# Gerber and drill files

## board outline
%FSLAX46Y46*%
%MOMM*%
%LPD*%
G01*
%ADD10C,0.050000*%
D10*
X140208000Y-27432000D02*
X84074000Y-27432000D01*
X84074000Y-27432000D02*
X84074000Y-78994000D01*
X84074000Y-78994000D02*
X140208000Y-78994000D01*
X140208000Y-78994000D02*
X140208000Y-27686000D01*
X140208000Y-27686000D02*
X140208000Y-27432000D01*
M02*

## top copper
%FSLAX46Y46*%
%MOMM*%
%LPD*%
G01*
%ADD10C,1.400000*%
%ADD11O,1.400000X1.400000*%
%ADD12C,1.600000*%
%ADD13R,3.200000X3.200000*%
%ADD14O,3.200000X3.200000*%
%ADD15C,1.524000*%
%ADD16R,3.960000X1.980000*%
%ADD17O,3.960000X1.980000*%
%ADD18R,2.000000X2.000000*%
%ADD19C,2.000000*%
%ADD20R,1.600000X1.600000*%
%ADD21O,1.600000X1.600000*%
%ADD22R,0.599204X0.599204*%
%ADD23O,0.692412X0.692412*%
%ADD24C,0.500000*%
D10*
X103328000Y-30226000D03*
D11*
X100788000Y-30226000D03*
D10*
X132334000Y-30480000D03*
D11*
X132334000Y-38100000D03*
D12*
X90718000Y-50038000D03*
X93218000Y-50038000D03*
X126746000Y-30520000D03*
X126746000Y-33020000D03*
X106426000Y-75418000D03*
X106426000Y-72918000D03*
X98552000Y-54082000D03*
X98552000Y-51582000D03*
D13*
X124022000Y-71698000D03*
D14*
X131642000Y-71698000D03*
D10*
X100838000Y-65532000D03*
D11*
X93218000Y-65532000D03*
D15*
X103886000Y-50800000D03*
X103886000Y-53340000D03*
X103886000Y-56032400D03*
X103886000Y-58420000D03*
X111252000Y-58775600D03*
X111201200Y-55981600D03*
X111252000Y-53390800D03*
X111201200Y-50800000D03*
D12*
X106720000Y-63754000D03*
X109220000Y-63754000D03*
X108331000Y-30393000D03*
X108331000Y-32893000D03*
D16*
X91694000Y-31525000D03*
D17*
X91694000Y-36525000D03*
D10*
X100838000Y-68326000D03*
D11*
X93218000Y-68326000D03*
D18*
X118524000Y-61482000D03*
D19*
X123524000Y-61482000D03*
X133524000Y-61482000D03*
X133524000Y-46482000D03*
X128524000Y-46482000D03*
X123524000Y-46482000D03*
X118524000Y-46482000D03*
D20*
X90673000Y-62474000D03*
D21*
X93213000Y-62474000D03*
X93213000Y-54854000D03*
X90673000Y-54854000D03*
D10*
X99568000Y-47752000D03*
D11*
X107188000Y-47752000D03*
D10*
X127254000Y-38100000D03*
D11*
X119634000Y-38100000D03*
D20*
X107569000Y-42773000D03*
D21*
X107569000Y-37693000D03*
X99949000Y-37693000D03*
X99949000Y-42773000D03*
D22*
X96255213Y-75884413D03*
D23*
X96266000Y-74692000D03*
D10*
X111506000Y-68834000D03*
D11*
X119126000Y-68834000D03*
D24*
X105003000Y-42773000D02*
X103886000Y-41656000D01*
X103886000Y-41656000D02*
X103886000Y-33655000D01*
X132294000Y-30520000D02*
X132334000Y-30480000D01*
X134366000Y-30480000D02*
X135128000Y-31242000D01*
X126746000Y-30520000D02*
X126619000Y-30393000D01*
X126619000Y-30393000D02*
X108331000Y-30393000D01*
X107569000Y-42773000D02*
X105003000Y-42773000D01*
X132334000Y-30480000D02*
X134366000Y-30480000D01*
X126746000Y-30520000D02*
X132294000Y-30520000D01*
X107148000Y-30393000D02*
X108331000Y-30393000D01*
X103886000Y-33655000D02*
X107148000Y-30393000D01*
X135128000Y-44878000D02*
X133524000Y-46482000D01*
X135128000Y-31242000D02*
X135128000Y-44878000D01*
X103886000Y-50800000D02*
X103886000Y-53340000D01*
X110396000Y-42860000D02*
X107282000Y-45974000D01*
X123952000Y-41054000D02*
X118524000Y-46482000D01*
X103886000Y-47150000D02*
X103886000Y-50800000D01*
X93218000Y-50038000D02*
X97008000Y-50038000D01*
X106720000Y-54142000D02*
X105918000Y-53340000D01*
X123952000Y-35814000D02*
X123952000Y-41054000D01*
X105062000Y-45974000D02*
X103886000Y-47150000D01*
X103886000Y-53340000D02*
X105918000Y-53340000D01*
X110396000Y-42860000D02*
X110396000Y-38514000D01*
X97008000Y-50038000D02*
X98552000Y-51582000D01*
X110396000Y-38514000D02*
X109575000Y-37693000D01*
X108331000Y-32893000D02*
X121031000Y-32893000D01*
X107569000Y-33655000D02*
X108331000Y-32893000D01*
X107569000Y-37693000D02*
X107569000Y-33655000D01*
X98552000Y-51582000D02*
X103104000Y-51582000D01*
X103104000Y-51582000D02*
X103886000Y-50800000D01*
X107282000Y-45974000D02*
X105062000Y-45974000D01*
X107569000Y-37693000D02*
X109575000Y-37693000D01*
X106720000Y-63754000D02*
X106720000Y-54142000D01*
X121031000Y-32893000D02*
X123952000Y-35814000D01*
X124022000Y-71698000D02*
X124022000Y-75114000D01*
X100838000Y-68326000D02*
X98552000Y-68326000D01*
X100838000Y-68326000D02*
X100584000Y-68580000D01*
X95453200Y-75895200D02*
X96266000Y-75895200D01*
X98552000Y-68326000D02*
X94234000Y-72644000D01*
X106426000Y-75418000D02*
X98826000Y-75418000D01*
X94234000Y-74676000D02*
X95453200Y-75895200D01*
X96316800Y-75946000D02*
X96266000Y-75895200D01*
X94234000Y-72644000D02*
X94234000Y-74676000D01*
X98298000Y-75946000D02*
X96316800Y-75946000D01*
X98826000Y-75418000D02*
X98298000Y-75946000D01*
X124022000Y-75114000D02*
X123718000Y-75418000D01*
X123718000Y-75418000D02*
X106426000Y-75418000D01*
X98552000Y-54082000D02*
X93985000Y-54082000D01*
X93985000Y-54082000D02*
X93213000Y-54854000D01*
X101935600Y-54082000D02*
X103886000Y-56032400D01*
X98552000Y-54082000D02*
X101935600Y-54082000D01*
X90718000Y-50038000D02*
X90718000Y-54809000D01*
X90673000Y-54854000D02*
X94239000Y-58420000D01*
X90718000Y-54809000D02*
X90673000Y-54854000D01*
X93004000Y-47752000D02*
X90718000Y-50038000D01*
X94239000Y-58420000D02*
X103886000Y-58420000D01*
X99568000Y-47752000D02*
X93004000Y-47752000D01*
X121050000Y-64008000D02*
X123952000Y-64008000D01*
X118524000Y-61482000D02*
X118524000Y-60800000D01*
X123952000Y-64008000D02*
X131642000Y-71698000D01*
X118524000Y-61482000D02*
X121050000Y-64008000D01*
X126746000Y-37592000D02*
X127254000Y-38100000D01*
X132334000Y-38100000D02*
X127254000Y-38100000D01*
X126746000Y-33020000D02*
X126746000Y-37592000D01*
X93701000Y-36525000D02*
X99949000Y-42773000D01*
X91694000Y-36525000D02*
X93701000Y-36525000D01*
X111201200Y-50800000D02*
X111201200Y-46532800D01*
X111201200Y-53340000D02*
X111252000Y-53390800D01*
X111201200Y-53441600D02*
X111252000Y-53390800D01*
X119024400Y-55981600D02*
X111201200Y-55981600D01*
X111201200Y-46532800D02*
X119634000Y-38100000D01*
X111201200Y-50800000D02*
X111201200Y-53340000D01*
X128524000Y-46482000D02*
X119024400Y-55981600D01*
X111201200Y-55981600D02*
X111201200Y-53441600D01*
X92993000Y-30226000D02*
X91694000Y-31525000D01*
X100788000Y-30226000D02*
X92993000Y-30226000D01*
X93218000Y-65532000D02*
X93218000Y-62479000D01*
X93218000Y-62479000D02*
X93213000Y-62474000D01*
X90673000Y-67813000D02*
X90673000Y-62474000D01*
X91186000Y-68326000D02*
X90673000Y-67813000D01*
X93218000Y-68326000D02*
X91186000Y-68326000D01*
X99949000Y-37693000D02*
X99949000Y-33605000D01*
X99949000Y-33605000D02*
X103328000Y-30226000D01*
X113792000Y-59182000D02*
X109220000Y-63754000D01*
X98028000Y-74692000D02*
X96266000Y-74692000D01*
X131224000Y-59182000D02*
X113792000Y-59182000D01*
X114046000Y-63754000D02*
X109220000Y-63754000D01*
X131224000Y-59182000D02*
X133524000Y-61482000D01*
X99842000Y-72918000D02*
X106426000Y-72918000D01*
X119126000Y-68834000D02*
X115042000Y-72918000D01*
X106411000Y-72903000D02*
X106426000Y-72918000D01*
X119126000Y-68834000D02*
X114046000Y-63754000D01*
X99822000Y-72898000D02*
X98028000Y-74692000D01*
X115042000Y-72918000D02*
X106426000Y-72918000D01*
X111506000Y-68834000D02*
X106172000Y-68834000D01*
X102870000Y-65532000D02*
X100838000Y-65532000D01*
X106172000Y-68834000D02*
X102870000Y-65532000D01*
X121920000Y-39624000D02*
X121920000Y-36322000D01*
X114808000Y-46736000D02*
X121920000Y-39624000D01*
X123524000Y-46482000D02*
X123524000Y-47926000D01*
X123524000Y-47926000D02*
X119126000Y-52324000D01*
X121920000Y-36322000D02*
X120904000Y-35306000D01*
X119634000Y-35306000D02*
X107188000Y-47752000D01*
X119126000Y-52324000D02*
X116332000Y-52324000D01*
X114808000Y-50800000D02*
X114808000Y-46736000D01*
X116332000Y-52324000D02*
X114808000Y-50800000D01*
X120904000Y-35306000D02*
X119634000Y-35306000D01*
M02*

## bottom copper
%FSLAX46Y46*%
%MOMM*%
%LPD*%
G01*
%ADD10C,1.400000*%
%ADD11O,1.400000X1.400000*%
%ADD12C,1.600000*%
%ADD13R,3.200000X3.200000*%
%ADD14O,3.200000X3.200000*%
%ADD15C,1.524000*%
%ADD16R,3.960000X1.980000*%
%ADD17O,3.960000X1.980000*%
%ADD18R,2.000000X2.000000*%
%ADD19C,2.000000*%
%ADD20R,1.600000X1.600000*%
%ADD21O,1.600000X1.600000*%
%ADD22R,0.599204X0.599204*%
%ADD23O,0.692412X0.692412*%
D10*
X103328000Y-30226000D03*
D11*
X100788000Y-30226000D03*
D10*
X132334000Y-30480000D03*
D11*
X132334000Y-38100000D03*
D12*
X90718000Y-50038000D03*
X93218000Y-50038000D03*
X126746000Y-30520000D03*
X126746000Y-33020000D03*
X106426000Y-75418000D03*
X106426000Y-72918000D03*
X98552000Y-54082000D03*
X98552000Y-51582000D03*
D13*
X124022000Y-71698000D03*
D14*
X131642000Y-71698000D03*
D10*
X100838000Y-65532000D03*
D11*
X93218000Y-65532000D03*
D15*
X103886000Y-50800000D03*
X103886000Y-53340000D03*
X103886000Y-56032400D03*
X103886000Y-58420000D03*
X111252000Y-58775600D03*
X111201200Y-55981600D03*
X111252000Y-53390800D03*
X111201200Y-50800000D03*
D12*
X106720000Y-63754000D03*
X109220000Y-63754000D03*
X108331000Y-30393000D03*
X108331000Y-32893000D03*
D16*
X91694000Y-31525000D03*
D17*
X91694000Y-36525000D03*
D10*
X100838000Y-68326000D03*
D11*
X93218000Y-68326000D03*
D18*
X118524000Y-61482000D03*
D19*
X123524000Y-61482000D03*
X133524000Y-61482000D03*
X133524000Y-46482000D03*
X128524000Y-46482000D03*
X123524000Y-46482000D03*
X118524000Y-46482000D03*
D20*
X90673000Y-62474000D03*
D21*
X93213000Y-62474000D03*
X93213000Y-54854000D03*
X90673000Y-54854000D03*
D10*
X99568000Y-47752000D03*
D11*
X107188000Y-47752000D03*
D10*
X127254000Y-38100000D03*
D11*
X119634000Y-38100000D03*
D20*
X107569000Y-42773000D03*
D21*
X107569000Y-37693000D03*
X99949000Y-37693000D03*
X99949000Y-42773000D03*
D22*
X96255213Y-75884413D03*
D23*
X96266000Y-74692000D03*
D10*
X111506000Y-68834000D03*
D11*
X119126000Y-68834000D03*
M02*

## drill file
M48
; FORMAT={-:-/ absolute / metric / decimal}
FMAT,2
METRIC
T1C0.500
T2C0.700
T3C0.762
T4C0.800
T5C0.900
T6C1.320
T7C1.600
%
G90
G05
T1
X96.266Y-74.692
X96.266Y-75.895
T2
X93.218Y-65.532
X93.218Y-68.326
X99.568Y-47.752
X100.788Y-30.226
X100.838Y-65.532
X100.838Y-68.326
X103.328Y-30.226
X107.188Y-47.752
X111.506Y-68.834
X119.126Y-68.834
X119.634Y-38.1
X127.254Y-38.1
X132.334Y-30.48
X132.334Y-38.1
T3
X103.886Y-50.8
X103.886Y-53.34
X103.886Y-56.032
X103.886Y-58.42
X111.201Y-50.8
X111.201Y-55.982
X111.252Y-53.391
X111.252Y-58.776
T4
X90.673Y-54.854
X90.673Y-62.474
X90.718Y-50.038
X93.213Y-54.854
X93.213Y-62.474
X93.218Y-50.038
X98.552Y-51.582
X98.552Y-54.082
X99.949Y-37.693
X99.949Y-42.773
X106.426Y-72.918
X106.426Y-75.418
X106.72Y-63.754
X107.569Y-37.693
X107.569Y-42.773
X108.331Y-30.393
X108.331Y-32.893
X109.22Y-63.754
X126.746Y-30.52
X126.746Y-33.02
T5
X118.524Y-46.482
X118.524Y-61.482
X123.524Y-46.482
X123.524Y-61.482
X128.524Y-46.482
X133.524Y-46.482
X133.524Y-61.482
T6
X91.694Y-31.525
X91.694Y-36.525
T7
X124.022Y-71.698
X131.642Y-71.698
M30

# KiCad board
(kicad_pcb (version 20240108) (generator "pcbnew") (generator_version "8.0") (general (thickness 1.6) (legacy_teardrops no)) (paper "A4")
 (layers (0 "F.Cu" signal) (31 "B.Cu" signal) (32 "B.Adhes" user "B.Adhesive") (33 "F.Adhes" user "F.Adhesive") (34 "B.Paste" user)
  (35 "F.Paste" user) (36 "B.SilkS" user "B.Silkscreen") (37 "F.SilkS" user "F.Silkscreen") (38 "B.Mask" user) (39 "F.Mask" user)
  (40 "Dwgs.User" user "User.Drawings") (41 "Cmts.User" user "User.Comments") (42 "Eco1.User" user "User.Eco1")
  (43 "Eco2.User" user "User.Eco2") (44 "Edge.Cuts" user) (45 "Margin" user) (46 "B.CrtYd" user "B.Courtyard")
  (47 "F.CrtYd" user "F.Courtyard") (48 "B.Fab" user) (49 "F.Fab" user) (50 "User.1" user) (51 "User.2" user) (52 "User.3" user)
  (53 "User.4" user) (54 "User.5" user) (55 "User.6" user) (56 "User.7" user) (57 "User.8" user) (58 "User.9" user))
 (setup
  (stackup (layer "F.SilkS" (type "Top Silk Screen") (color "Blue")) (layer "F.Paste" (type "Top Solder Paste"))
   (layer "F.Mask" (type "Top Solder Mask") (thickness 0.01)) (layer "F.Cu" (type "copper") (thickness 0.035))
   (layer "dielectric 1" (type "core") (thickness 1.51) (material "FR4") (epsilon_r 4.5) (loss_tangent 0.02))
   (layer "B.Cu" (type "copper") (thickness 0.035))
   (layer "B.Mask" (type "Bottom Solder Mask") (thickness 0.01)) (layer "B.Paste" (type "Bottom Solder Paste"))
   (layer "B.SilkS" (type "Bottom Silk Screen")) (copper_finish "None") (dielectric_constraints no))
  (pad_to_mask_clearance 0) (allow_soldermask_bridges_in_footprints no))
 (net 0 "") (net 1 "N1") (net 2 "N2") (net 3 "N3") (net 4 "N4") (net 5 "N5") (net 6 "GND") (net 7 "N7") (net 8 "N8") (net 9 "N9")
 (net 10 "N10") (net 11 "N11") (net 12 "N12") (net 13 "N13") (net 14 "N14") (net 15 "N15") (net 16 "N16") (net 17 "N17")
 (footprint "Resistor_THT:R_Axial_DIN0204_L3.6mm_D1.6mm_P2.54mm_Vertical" (layer "F.Cu") (at 103.328 30.226 180)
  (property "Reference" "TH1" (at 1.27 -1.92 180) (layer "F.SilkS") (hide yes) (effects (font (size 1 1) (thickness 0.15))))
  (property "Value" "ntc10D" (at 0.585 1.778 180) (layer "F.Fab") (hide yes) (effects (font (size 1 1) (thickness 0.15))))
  (pad "1" thru_hole circle (at 0 0 180) (size 1.4 1.4) (drill 0.7) (layers "*.Cu" "*.Mask") (remove_unused_layers no) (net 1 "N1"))
  (pad "2" thru_hole oval (at 2.54 0 180) (size 1.4 1.4) (drill 0.7) (layers "*.Cu" "*.Mask") (remove_unused_layers no) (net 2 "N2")))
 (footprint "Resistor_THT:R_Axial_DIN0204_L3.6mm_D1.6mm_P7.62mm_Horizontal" (layer "F.Cu") (at 132.334 30.48 -90)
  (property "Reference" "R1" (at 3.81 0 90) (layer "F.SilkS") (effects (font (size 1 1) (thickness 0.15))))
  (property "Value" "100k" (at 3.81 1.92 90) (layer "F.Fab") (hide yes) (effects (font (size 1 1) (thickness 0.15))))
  (pad "1" thru_hole circle (at 0 0 270) (size 1.4 1.4) (drill 0.7) (layers "*.Cu" "*.Mask") (remove_unused_layers no) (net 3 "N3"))
  (pad "2" thru_hole oval (at 7.62 0 270) (size 1.4 1.4) (drill 0.7) (layers "*.Cu" "*.Mask") (remove_unused_layers no) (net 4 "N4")))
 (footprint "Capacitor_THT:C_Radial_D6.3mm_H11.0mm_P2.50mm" (layer "F.Cu") (at 90.718 50.038)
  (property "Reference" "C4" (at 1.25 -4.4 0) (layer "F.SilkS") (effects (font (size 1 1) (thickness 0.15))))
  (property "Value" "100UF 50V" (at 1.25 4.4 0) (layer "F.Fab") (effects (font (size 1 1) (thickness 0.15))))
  (pad "1" thru_hole circle (at 0 0) (size 1.6 1.6) (drill 0.8) (layers "*.Cu" "*.Mask") (remove_unused_layers no) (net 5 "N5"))
  (pad "2" thru_hole circle (at 2.5 0) (size 1.6 1.6) (drill 0.8) (layers "*.Cu" "*.Mask") (remove_unused_layers no) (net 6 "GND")))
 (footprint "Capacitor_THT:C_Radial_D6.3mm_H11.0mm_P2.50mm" (layer "F.Cu") (at 126.746 30.52 -90)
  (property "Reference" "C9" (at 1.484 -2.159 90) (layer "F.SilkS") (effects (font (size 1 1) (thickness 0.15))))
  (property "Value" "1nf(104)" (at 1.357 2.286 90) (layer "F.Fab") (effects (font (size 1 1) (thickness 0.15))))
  (pad "1" thru_hole circle (at 0 0 270) (size 1.6 1.6) (drill 0.8) (layers "*.Cu" "*.Mask") (remove_unused_layers no) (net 3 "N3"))
  (pad "2" thru_hole circle (at 2.5 0 270) (size 1.6 1.6) (drill 0.8) (layers "*.Cu" "*.Mask") (remove_unused_layers no) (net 4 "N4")))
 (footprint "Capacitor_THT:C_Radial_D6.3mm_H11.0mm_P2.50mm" (layer "F.Cu") (at 106.426 75.418 90)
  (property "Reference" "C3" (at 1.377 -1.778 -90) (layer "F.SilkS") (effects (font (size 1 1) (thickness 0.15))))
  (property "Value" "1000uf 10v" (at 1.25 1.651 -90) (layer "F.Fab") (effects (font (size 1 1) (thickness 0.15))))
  (pad "1" thru_hole circle (at 0 0 90) (size 1.6 1.6) (drill 0.8) (layers "*.Cu" "*.Mask") (remove_unused_layers no) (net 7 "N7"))
  (pad "2" thru_hole circle (at 2.5 0 90) (size 1.6 1.6) (drill 0.8) (layers "*.Cu" "*.Mask") (remove_unused_layers no) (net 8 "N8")))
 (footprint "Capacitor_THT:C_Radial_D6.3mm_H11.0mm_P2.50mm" (layer "F.Cu") (at 98.552 54.082 90)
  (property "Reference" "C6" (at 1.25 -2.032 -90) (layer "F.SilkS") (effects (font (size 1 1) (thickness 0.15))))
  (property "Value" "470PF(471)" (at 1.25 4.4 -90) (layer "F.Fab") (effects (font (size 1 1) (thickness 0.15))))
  (pad "1" thru_hole circle (at 0 0 90) (size 1.6 1.6) (drill 0.8) (layers "*.Cu" "*.Mask") (remove_unused_layers no) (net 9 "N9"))
  (pad "2" thru_hole circle (at 2.5 0 90) (size 1.6 1.6) (drill 0.8) (layers "*.Cu" "*.Mask") (remove_unused_layers no) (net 6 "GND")))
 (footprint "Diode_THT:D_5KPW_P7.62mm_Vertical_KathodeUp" (layer "F.Cu") (at 124.022 71.698)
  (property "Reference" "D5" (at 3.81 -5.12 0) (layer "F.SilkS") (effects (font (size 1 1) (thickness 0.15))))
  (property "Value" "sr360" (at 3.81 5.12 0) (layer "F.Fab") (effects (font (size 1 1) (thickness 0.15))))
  (pad "1" thru_hole rect (at 0 0) (size 3.2 3.2) (drill 1.6) (layers "*.Cu" "*.Mask") (remove_unused_layers no) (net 7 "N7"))
  (pad "2" thru_hole oval (at 7.62 0) (size 3.2 3.2) (drill 1.6) (layers "*.Cu" "*.Mask") (remove_unused_layers no) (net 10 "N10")))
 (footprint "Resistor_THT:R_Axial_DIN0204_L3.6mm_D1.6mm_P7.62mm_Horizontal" (layer "F.Cu") (at 100.838 65.532 180)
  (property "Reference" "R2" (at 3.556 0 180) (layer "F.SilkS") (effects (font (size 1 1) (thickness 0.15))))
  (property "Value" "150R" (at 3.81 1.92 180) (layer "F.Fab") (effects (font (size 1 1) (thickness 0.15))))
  (pad "1" thru_hole circle (at 0 0 180) (size 1.4 1.4) (drill 0.7) (layers "*.Cu" "*.Mask") (remove_unused_layers no) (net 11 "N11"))
  (pad "2" thru_hole oval (at 7.62 0 180) (size 1.4 1.4) (drill 0.7) (layers "*.Cu" "*.Mask") (remove_unused_layers no) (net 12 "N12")))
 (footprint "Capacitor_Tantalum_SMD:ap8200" (layer "F.Cu") (at 107.5436 54.6608)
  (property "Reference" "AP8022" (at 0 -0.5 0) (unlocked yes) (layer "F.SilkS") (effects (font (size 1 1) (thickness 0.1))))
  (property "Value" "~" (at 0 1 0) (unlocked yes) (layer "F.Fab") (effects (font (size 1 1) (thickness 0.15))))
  (pad "1" thru_hole circle (at -3.6576 -3.8608) (size 1.524 1.524) (drill 0.762) (layers "*.Cu" "*.Mask") (remove_unused_layers no)
   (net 6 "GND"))
  (pad "2" thru_hole circle (at -3.6576 -1.3208) (size 1.524 1.524) (drill 0.762) (layers "*.Cu" "*.Mask") (remove_unused_layers no)
   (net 6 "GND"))
  (pad "3" thru_hole circle (at -3.6576 1.3716) (size 1.524 1.524) (drill 0.762) (layers "*.Cu" "*.Mask") (remove_unused_layers no)
   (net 9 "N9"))
  (pad "4" thru_hole circle (at -3.6576 3.7592) (size 1.524 1.524) (drill 0.762) (layers "*.Cu" "*.Mask") (remove_unused_layers no)
   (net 5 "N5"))
  (pad "5" thru_hole circle (at 3.7084 4.1148) (size 1.524 1.524) (drill 0.762) (layers "*.Cu" "*.Mask") (remove_unused_layers no)
   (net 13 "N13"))
  (pad "6" thru_hole circle (at 3.6576 1.3208) (size 1.524 1.524) (drill 0.762) (layers "*.Cu" "*.Mask") (remove_unused_layers no)
   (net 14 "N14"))
  (pad "7" thru_hole circle (at 3.7084 -1.27) (size 1.524 1.524) (drill 0.762) (layers "*.Cu" "*.Mask") (remove_unused_layers no)
   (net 14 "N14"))
  (pad "8" thru_hole circle (at 3.6576 -3.8608) (size 1.524 1.524) (drill 0.762) (layers "*.Cu" "*.Mask") (remove_unused_layers no)
   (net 14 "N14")))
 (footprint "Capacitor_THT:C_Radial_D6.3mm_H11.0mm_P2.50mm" (layer "F.Cu") (at 106.72 63.754)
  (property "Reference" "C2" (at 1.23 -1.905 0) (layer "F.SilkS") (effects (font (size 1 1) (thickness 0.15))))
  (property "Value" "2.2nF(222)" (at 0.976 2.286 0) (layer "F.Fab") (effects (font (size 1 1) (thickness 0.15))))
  (pad "1" thru_hole circle (at 0 0) (size 1.6 1.6) (drill 0.8) (layers "*.Cu" "*.Mask") (remove_unused_layers no) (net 6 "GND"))
  (pad "2" thru_hole circle (at 2.5 0) (size 1.6 1.6) (drill 0.8) (layers "*.Cu" "*.Mask") (remove_unused_layers no) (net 8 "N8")))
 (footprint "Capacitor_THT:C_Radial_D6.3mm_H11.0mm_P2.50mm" (layer "F.Cu") (at 108.331 30.393 -90)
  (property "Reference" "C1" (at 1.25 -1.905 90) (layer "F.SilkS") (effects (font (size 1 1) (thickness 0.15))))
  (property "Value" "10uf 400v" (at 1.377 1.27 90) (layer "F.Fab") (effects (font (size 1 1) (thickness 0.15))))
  (pad "1" thru_hole circle (at 0 0 270) (size 1.6 1.6) (drill 0.8) (layers "*.Cu" "*.Mask") (remove_unused_layers no) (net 3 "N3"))
  (pad "2" thru_hole circle (at 2.5 0 270) (size 1.6 1.6) (drill 0.8) (layers "*.Cu" "*.Mask") (remove_unused_layers no) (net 6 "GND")))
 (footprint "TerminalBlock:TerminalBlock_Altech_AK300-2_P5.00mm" (layer "F.Cu") (at 91.694 31.525 -90)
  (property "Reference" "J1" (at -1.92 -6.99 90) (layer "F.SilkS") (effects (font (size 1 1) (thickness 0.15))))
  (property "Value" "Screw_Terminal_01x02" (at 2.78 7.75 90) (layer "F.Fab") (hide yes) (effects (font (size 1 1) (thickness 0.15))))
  (pad "1" thru_hole rect (at 0 0 270) (size 1.98 3.96) (drill 1.32) (layers "*.Cu" "*.Mask") (remove_unused_layers no) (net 2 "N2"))
  (pad "2" thru_hole oval (at 5 0 270) (size 1.98 3.96) (drill 1.32) (layers "*.Cu" "*.Mask") (remove_unused_layers no) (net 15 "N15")))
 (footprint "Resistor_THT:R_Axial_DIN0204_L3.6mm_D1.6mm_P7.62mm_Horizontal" (layer "F.Cu") (at 100.838 68.326 180)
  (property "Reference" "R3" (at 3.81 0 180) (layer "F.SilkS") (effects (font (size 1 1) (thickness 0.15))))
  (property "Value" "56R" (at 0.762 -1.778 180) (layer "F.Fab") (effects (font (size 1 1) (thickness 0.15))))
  (pad "1" thru_hole circle (at 0 0 180) (size 1.4 1.4) (drill 0.7) (layers "*.Cu" "*.Mask") (remove_unused_layers no) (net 7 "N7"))
  (pad "2" thru_hole oval (at 7.62 0 180) (size 1.4 1.4) (drill 0.7) (layers "*.Cu" "*.Mask") (remove_unused_layers no) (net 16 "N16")))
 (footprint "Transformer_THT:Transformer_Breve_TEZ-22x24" (layer "F.Cu") (at 118.524 61.482)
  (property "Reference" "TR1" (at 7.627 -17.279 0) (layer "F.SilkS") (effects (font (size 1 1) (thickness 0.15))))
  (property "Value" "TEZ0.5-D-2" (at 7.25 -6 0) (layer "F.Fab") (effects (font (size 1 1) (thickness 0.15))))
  (pad "1" thru_hole rect (at 0 0) (size 2 2) (drill 0.9) (layers "*.Cu" "*.Mask") (remove_unused_layers no) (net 10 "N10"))
  (pad "2" thru_hole circle (at 5 0) (size 2 2) (drill 0.9) (layers "*.Cu" "*.Mask") (remove_unused_layers no))
  (pad "4" thru_hole circle (at 15 0) (size 2 2) (drill 0.9) (layers "*.Cu" "*.Mask") (remove_unused_layers no) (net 8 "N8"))
  (pad "5" thru_hole circle (at 15 -15) (size 2 2) (drill 0.9) (layers "*.Cu" "*.Mask") (remove_unused_layers no) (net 3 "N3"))
  (pad "6" thru_hole circle (at 10 -15) (size 2 2) (drill 0.9) (layers "*.Cu" "*.Mask") (remove_unused_layers no) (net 14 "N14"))
  (pad "7" thru_hole circle (at 5 -15) (size 2 2) (drill 0.9) (layers "*.Cu" "*.Mask") (remove_unused_layers no) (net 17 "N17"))
  (pad "8" thru_hole circle (at 0 -15) (size 2 2) (drill 0.9) (layers "*.Cu" "*.Mask") (remove_unused_layers no) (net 6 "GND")))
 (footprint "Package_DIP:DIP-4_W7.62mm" (layer "F.Cu") (at 90.673 62.474 90)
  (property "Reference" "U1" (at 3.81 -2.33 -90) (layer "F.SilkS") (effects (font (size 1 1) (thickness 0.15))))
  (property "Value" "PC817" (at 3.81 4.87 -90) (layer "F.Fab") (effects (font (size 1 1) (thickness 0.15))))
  (pad "1" thru_hole rect (at 0 0 90) (size 1.6 1.6) (drill 0.8) (layers "*.Cu" "*.Mask") (remove_unused_layers no) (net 16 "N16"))
  (pad "2" thru_hole oval (at 0 2.54 90) (size 1.6 1.6) (drill 0.8) (layers "*.Cu" "*.Mask") (remove_unused_layers no) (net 12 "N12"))
  (pad "3" thru_hole oval (at 7.62 2.54 90) (size 1.6 1.6) (drill 0.8) (layers "*.Cu" "*.Mask") (remove_unused_layers no) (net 9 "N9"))
  (pad "4" thru_hole oval (at 7.62 0 90) (size 1.6 1.6) (drill 0.8) (layers "*.Cu" "*.Mask") (remove_unused_layers no) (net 5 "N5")))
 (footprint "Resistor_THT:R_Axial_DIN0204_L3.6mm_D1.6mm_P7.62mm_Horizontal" (layer "F.Cu") (at 99.568 47.752)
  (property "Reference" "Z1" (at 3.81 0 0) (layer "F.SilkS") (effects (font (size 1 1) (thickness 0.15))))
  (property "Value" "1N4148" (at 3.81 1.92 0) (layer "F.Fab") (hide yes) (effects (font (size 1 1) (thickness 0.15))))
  (pad "1" thru_hole circle (at 0 0) (size 1.4 1.4) (drill 0.7) (layers "*.Cu" "*.Mask") (remove_unused_layers no) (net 5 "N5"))
  (pad "2" thru_hole oval (at 7.62 0) (size 1.4 1.4) (drill 0.7) (layers "*.Cu" "*.Mask") (remove_unused_layers no) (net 17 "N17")))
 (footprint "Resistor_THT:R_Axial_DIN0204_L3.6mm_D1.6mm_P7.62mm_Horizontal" (layer "F.Cu") (at 127.254 38.1 180)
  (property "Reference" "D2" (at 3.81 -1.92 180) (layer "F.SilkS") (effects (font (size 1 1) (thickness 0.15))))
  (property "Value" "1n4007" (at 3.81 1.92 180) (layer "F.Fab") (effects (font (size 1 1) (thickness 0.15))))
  (pad "1" thru_hole circle (at 0 0 180) (size 1.4 1.4) (drill 0.7) (layers "*.Cu" "*.Mask") (remove_unused_layers no) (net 4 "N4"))
  (pad "2" thru_hole oval (at 7.62 0 180) (size 1.4 1.4) (drill 0.7) (layers "*.Cu" "*.Mask") (remove_unused_layers no) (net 14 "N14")))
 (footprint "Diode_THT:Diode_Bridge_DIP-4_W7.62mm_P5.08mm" (layer "F.Cu") (at 107.569 42.773 180)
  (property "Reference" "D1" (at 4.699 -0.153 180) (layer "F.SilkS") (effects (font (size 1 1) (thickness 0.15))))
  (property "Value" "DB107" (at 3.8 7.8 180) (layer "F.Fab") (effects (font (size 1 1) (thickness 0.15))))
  (pad "1" thru_hole rect (at 0 0 180) (size 1.6 1.6) (drill 0.8) (layers "*.Cu" "*.Mask") (remove_unused_layers no) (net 3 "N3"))
  (pad "2" thru_hole oval (at 0 5.08 180) (size 1.6 1.6) (drill 0.8) (layers "*.Cu" "*.Mask") (remove_unused_layers no) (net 6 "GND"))
  (pad "3" thru_hole oval (at 7.62 5.08 180) (size 1.6 1.6) (drill 0.8) (layers "*.Cu" "*.Mask") (remove_unused_layers no) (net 1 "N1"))
  (pad "4" thru_hole oval (at 7.62 0 180) (size 1.6 1.6) (drill 0.8) (layers "*.Cu" "*.Mask") (remove_unused_layers no) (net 15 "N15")))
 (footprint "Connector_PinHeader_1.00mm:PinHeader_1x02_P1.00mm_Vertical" (layer "F.Cu") (at 96.266 75.692 180)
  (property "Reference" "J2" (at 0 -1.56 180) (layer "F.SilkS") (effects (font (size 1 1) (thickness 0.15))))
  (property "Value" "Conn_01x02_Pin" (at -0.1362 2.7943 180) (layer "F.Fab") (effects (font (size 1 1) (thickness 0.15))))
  (pad "1" thru_hole rect (at 0 -0.2032 180) (size 0.599204 0.599204) (drill 0.5 (offset 0.010787 0.010787)) (layers "*.Cu" "*.Mask")
   (remove_unused_layers no) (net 7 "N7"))
  (pad "2" thru_hole oval (at 0 1 180) (size 0.692412 0.692412) (drill 0.5) (layers "*.Cu" "*.Mask") (remove_unused_layers no) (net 8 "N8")))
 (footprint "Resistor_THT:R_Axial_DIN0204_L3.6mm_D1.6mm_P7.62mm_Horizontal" (layer "F.Cu") (at 111.506 68.834)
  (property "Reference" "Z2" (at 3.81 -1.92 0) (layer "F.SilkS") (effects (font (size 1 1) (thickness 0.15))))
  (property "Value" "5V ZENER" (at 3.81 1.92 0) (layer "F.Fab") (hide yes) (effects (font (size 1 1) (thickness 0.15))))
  (pad "1" thru_hole circle (at 0 0) (size 1.4 1.4) (drill 0.7) (layers "*.Cu" "*.Mask") (remove_unused_layers no) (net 11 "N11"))
  (pad "2" thru_hole oval (at 7.62 0) (size 1.4 1.4) (drill 0.7) (layers "*.Cu" "*.Mask") (remove_unused_layers no) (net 8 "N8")))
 (gr_line (start 140.208 27.432) (end 84.074 27.432) (stroke (width 0.05) (type default)) (layer "Edge.Cuts"))
 (gr_line (start 84.074 27.432) (end 84.074 78.994) (stroke (width 0.05) (type default)) (layer "Edge.Cuts"))
 (gr_line (start 84.074 78.994) (end 140.208 78.994) (stroke (width 0.05) (type default)) (layer "Edge.Cuts"))
 (gr_line (start 140.208 78.994) (end 140.208 27.686) (stroke (width 0.05) (type default)) (layer "Edge.Cuts"))
 (gr_line (start 140.208 27.686) (end 140.208 27.432) (stroke (width 0.05) (type default)) (layer "Edge.Cuts"))
 (segment (start 105.003 42.773) (end 103.886 41.656) (width 0.5) (layer "F.Cu") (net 3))
 (segment (start 103.886 41.656) (end 103.886 33.655) (width 0.5) (layer "F.Cu") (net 3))
 (segment (start 132.294 30.52) (end 132.334 30.48) (width 0.5) (layer "F.Cu") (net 3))
 (segment (start 134.366 30.48) (end 135.128 31.242) (width 0.5) (layer "F.Cu") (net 3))
 (segment (start 126.746 30.52) (end 126.619 30.393) (width 0.5) (layer "F.Cu") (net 3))
 (segment (start 126.619 30.393) (end 108.331 30.393) (width 0.5) (layer "F.Cu") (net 3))
 (segment (start 107.569 42.773) (end 105.003 42.773) (width 0.5) (layer "F.Cu") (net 3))
 (segment (start 132.334 30.48) (end 134.366 30.48) (width 0.5) (layer "F.Cu") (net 3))
 (segment (start 126.746 30.52) (end 132.294 30.52) (width 0.5) (layer "F.Cu") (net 3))
 (segment (start 107.148 30.393) (end 108.331 30.393) (width 0.5) (layer "F.Cu") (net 3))
 (segment (start 103.886 33.655) (end 107.148 30.393) (width 0.5) (layer "F.Cu") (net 3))
 (segment (start 135.128 44.878) (end 133.524 46.482) (width 0.5) (layer "F.Cu") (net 3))
 (segment (start 135.128 31.242) (end 135.128 44.878) (width 0.5) (layer "F.Cu") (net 3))
 (segment (start 103.886 50.8) (end 103.886 53.34) (width 0.5) (layer "F.Cu") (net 6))
 (segment (start 110.396 42.86) (end 107.282 45.974) (width 0.5) (layer "F.Cu") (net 6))
 (segment (start 123.952 41.054) (end 118.524 46.482) (width 0.5) (layer "F.Cu") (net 6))
 (segment (start 103.886 47.15) (end 103.886 50.8) (width 0.5) (layer "F.Cu") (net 6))
 (segment (start 93.218 50.038) (end 97.008 50.038) (width 0.5) (layer "F.Cu") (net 6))
 (segment (start 106.72 54.142) (end 105.918 53.34) (width 0.5) (layer "F.Cu") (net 6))
 (segment (start 123.952 35.814) (end 123.952 41.054) (width 0.5) (layer "F.Cu") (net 6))
 (segment (start 105.062 45.974) (end 103.886 47.15) (width 0.5) (layer "F.Cu") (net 6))
 (segment (start 103.886 53.34) (end 105.918 53.34) (width 0.5) (layer "F.Cu") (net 6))
 (segment (start 110.396 42.86) (end 110.396 38.514) (width 0.5) (layer "F.Cu") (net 6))
 (segment (start 97.008 50.038) (end 98.552 51.582) (width 0.5) (layer "F.Cu") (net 6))
 (segment (start 110.396 38.514) (end 109.575 37.693) (width 0.5) (layer "F.Cu") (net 6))
 (segment (start 108.331 32.893) (end 121.031 32.893) (width 0.5) (layer "F.Cu") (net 6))
 (segment (start 107.569 33.655) (end 108.331 32.893) (width 0.5) (layer "F.Cu") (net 6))
 (segment (start 107.569 37.693) (end 107.569 33.655) (width 0.5) (layer "F.Cu") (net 6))
 (segment (start 98.552 51.582) (end 103.104 51.582) (width 0.5) (layer "F.Cu") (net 6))
 (segment (start 103.104 51.582) (end 103.886 50.8) (width 0.5) (layer "F.Cu") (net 6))
 (segment (start 107.282 45.974) (end 105.062 45.974) (width 0.5) (layer "F.Cu") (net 6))
 (segment (start 107.569 37.693) (end 109.575 37.693) (width 0.5) (layer "F.Cu") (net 6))
 (segment (start 106.72 63.754) (end 106.72 54.142) (width 0.5) (layer "F.Cu") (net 6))
 (segment (start 121.031 32.893) (end 123.952 35.814) (width 0.5) (layer "F.Cu") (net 6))
 (segment (start 124.022 71.698) (end 124.022 75.114) (width 0.5) (layer "F.Cu") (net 7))
 (segment (start 100.838 68.326) (end 98.552 68.326) (width 0.5) (layer "F.Cu") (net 7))
 (segment (start 100.838 68.326) (end 100.584 68.58) (width 0.5) (layer "F.Cu") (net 7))
 (segment (start 95.4532 75.8952) (end 96.266 75.8952) (width 0.5) (layer "F.Cu") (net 7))
 (segment (start 98.552 68.326) (end 94.234 72.644) (width 0.5) (layer "F.Cu") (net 7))
 (segment (start 106.426 75.418) (end 98.826 75.418) (width 0.5) (layer "F.Cu") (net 7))
 (segment (start 94.234 74.676) (end 95.4532 75.8952) (width 0.5) (layer "F.Cu") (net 7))
 (segment (start 96.3168 75.946) (end 96.266 75.8952) (width 0.5) (layer "F.Cu") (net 7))
 (segment (start 94.234 72.644) (end 94.234 74.676) (width 0.5) (layer "F.Cu") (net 7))
 (segment (start 98.298 75.946) (end 96.3168 75.946) (width 0.5) (layer "F.Cu") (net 7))
 (segment (start 98.826 75.418) (end 98.298 75.946) (width 0.5) (layer "F.Cu") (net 7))
 (segment (start 124.022 75.114) (end 123.718 75.418) (width 0.5) (layer "F.Cu") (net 7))
 (segment (start 123.718 75.418) (end 106.426 75.418) (width 0.5) (layer "F.Cu") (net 7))
 (segment (start 98.552 54.082) (end 93.985 54.082) (width 0.5) (layer "F.Cu") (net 9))
 (segment (start 93.985 54.082) (end 93.213 54.854) (width 0.5) (layer "F.Cu") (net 9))
 (segment (start 101.9356 54.082) (end 103.886 56.0324) (width 0.5) (layer "F.Cu") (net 9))
 (segment (start 98.552 54.082) (end 101.9356 54.082) (width 0.5) (layer "F.Cu") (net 9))
 (segment (start 90.718 50.038) (end 90.718 54.809) (width 0.5) (layer "F.Cu") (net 5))
 (segment (start 90.673 54.854) (end 94.239 58.42) (width 0.5) (layer "F.Cu") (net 5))
 (segment (start 90.718 54.809) (end 90.673 54.854) (width 0.5) (layer "F.Cu") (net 5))
 (segment (start 93.004 47.752) (end 90.718 50.038) (width 0.5) (layer "F.Cu") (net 5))
 (segment (start 94.239 58.42) (end 103.886 58.42) (width 0.5) (layer "F.Cu") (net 5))
 (segment (start 99.568 47.752) (end 93.004 47.752) (width 0.5) (layer "F.Cu") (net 5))
 (segment (start 121.05 64.008) (end 123.952 64.008) (width 0.5) (layer "F.Cu") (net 10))
 (segment (start 118.524 61.482) (end 118.524 60.8) (width 0.5) (layer "F.Cu") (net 10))
 (segment (start 123.952 64.008) (end 131.642 71.698) (width 0.5) (layer "F.Cu") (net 10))
 (segment (start 118.524 61.482) (end 121.05 64.008) (width 0.5) (layer "F.Cu") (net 10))
 (segment (start 126.746 37.592) (end 127.254 38.1) (width 0.5) (layer "F.Cu") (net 4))
 (segment (start 132.334 38.1) (end 127.254 38.1) (width 0.5) (layer "F.Cu") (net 4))
 (segment (start 126.746 33.02) (end 126.746 37.592) (width 0.5) (layer "F.Cu") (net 4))
 (segment (start 93.701 36.525) (end 99.949 42.773) (width 0.5) (layer "F.Cu") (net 15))
 (segment (start 91.694 36.525) (end 93.701 36.525) (width 0.5) (layer "F.Cu") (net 15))
 (segment (start 111.2012 50.8) (end 111.2012 46.5328) (width 0.5) (layer "F.Cu") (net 14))
 (segment (start 111.2012 53.34) (end 111.252 53.3908) (width 0.5) (layer "F.Cu") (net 14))
 (segment (start 111.2012 53.4416) (end 111.252 53.3908) (width 0.5) (layer "F.Cu") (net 14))
 (segment (start 119.0244 55.9816) (end 111.2012 55.9816) (width 0.5) (layer "F.Cu") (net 14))
 (segment (start 111.2012 46.5328) (end 119.634 38.1) (width 0.5) (layer "F.Cu") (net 14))
 (segment (start 111.2012 50.8) (end 111.2012 53.34) (width 0.5) (layer "F.Cu") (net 14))
 (segment (start 128.524 46.482) (end 119.0244 55.9816) (width 0.5) (layer "F.Cu") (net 14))
 (segment (start 111.2012 55.9816) (end 111.2012 53.4416) (width 0.5) (layer "F.Cu") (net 14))
 (segment (start 92.993 30.226) (end 91.694 31.525) (width 0.5) (layer "F.Cu") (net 2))
 (segment (start 100.788 30.226) (end 92.993 30.226) (width 0.5) (layer "F.Cu") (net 2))
 (segment (start 93.218 65.532) (end 93.218 62.479) (width 0.5) (layer "F.Cu") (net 12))
 (segment (start 93.218 62.479) (end 93.213 62.474) (width 0.5) (layer "F.Cu") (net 12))
 (segment (start 90.673 67.813) (end 90.673 62.474) (width 0.5) (layer "F.Cu") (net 16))
 (segment (start 91.186 68.326) (end 90.673 67.813) (width 0.5) (layer "F.Cu") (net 16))
 (segment (start 93.218 68.326) (end 91.186 68.326) (width 0.5) (layer "F.Cu") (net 16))
 (segment (start 99.949 37.693) (end 99.949 33.605) (width 0.5) (layer "F.Cu") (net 1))
 (segment (start 99.949 33.605) (end 103.328 30.226) (width 0.5) (layer "F.Cu") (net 1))
 (segment (start 113.792 59.182) (end 109.22 63.754) (width 0.5) (layer "F.Cu") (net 8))
 (segment (start 98.028 74.692) (end 96.266 74.692) (width 0.5) (layer "F.Cu") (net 8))
 (segment (start 131.224 59.182) (end 113.792 59.182) (width 0.5) (layer "F.Cu") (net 8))
 (segment (start 114.046 63.754) (end 109.22 63.754) (width 0.5) (layer "F.Cu") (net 8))
 (segment (start 131.224 59.182) (end 133.524 61.482) (width 0.5) (layer "F.Cu") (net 8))
 (segment (start 99.842 72.918) (end 106.426 72.918) (width 0.5) (layer "F.Cu") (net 8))
 (segment (start 119.126 68.834) (end 115.042 72.918) (width 0.5) (layer "F.Cu") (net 8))
 (segment (start 106.411 72.903) (end 106.426 72.918) (width 0.5) (layer "F.Cu") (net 8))
 (segment (start 119.126 68.834) (end 114.046 63.754) (width 0.5) (layer "F.Cu") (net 8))
 (segment (start 99.822 72.898) (end 98.028 74.692) (width 0.5) (layer "F.Cu") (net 8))
 (segment (start 115.042 72.918) (end 106.426 72.918) (width 0.5) (layer "F.Cu") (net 8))
 (segment (start 111.506 68.834) (end 106.172 68.834) (width 0.5) (layer "F.Cu") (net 11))
 (segment (start 102.87 65.532) (end 100.838 65.532) (width 0.5) (layer "F.Cu") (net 11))
 (segment (start 106.172 68.834) (end 102.87 65.532) (width 0.5) (layer "F.Cu") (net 11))
 (segment (start 121.92 39.624) (end 121.92 36.322) (width 0.5) (layer "F.Cu") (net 17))
 (segment (start 114.808 46.736) (end 121.92 39.624) (width 0.5) (layer "F.Cu") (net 17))
 (segment (start 123.524 46.482) (end 123.524 47.926) (width 0.5) (layer "F.Cu") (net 17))
 (segment (start 123.524 47.926) (end 119.126 52.324) (width 0.5) (layer "F.Cu") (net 17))
 (segment (start 121.92 36.322) (end 120.904 35.306) (width 0.5) (layer "F.Cu") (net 17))
 (segment (start 119.634 35.306) (end 107.188 47.752) (width 0.5) (layer "F.Cu") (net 17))
 (segment (start 119.126 52.324) (end 116.332 52.324) (width 0.5) (layer "F.Cu") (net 17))
 (segment (start 114.808 50.8) (end 114.808 46.736) (width 0.5) (layer "F.Cu") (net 17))
 (segment (start 116.332 52.324) (end 114.808 50.8) (width 0.5) (layer "F.Cu") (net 17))
 (segment (start 120.904 35.306) (end 119.634 35.306) (width 0.5) (layer "F.Cu") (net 17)))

